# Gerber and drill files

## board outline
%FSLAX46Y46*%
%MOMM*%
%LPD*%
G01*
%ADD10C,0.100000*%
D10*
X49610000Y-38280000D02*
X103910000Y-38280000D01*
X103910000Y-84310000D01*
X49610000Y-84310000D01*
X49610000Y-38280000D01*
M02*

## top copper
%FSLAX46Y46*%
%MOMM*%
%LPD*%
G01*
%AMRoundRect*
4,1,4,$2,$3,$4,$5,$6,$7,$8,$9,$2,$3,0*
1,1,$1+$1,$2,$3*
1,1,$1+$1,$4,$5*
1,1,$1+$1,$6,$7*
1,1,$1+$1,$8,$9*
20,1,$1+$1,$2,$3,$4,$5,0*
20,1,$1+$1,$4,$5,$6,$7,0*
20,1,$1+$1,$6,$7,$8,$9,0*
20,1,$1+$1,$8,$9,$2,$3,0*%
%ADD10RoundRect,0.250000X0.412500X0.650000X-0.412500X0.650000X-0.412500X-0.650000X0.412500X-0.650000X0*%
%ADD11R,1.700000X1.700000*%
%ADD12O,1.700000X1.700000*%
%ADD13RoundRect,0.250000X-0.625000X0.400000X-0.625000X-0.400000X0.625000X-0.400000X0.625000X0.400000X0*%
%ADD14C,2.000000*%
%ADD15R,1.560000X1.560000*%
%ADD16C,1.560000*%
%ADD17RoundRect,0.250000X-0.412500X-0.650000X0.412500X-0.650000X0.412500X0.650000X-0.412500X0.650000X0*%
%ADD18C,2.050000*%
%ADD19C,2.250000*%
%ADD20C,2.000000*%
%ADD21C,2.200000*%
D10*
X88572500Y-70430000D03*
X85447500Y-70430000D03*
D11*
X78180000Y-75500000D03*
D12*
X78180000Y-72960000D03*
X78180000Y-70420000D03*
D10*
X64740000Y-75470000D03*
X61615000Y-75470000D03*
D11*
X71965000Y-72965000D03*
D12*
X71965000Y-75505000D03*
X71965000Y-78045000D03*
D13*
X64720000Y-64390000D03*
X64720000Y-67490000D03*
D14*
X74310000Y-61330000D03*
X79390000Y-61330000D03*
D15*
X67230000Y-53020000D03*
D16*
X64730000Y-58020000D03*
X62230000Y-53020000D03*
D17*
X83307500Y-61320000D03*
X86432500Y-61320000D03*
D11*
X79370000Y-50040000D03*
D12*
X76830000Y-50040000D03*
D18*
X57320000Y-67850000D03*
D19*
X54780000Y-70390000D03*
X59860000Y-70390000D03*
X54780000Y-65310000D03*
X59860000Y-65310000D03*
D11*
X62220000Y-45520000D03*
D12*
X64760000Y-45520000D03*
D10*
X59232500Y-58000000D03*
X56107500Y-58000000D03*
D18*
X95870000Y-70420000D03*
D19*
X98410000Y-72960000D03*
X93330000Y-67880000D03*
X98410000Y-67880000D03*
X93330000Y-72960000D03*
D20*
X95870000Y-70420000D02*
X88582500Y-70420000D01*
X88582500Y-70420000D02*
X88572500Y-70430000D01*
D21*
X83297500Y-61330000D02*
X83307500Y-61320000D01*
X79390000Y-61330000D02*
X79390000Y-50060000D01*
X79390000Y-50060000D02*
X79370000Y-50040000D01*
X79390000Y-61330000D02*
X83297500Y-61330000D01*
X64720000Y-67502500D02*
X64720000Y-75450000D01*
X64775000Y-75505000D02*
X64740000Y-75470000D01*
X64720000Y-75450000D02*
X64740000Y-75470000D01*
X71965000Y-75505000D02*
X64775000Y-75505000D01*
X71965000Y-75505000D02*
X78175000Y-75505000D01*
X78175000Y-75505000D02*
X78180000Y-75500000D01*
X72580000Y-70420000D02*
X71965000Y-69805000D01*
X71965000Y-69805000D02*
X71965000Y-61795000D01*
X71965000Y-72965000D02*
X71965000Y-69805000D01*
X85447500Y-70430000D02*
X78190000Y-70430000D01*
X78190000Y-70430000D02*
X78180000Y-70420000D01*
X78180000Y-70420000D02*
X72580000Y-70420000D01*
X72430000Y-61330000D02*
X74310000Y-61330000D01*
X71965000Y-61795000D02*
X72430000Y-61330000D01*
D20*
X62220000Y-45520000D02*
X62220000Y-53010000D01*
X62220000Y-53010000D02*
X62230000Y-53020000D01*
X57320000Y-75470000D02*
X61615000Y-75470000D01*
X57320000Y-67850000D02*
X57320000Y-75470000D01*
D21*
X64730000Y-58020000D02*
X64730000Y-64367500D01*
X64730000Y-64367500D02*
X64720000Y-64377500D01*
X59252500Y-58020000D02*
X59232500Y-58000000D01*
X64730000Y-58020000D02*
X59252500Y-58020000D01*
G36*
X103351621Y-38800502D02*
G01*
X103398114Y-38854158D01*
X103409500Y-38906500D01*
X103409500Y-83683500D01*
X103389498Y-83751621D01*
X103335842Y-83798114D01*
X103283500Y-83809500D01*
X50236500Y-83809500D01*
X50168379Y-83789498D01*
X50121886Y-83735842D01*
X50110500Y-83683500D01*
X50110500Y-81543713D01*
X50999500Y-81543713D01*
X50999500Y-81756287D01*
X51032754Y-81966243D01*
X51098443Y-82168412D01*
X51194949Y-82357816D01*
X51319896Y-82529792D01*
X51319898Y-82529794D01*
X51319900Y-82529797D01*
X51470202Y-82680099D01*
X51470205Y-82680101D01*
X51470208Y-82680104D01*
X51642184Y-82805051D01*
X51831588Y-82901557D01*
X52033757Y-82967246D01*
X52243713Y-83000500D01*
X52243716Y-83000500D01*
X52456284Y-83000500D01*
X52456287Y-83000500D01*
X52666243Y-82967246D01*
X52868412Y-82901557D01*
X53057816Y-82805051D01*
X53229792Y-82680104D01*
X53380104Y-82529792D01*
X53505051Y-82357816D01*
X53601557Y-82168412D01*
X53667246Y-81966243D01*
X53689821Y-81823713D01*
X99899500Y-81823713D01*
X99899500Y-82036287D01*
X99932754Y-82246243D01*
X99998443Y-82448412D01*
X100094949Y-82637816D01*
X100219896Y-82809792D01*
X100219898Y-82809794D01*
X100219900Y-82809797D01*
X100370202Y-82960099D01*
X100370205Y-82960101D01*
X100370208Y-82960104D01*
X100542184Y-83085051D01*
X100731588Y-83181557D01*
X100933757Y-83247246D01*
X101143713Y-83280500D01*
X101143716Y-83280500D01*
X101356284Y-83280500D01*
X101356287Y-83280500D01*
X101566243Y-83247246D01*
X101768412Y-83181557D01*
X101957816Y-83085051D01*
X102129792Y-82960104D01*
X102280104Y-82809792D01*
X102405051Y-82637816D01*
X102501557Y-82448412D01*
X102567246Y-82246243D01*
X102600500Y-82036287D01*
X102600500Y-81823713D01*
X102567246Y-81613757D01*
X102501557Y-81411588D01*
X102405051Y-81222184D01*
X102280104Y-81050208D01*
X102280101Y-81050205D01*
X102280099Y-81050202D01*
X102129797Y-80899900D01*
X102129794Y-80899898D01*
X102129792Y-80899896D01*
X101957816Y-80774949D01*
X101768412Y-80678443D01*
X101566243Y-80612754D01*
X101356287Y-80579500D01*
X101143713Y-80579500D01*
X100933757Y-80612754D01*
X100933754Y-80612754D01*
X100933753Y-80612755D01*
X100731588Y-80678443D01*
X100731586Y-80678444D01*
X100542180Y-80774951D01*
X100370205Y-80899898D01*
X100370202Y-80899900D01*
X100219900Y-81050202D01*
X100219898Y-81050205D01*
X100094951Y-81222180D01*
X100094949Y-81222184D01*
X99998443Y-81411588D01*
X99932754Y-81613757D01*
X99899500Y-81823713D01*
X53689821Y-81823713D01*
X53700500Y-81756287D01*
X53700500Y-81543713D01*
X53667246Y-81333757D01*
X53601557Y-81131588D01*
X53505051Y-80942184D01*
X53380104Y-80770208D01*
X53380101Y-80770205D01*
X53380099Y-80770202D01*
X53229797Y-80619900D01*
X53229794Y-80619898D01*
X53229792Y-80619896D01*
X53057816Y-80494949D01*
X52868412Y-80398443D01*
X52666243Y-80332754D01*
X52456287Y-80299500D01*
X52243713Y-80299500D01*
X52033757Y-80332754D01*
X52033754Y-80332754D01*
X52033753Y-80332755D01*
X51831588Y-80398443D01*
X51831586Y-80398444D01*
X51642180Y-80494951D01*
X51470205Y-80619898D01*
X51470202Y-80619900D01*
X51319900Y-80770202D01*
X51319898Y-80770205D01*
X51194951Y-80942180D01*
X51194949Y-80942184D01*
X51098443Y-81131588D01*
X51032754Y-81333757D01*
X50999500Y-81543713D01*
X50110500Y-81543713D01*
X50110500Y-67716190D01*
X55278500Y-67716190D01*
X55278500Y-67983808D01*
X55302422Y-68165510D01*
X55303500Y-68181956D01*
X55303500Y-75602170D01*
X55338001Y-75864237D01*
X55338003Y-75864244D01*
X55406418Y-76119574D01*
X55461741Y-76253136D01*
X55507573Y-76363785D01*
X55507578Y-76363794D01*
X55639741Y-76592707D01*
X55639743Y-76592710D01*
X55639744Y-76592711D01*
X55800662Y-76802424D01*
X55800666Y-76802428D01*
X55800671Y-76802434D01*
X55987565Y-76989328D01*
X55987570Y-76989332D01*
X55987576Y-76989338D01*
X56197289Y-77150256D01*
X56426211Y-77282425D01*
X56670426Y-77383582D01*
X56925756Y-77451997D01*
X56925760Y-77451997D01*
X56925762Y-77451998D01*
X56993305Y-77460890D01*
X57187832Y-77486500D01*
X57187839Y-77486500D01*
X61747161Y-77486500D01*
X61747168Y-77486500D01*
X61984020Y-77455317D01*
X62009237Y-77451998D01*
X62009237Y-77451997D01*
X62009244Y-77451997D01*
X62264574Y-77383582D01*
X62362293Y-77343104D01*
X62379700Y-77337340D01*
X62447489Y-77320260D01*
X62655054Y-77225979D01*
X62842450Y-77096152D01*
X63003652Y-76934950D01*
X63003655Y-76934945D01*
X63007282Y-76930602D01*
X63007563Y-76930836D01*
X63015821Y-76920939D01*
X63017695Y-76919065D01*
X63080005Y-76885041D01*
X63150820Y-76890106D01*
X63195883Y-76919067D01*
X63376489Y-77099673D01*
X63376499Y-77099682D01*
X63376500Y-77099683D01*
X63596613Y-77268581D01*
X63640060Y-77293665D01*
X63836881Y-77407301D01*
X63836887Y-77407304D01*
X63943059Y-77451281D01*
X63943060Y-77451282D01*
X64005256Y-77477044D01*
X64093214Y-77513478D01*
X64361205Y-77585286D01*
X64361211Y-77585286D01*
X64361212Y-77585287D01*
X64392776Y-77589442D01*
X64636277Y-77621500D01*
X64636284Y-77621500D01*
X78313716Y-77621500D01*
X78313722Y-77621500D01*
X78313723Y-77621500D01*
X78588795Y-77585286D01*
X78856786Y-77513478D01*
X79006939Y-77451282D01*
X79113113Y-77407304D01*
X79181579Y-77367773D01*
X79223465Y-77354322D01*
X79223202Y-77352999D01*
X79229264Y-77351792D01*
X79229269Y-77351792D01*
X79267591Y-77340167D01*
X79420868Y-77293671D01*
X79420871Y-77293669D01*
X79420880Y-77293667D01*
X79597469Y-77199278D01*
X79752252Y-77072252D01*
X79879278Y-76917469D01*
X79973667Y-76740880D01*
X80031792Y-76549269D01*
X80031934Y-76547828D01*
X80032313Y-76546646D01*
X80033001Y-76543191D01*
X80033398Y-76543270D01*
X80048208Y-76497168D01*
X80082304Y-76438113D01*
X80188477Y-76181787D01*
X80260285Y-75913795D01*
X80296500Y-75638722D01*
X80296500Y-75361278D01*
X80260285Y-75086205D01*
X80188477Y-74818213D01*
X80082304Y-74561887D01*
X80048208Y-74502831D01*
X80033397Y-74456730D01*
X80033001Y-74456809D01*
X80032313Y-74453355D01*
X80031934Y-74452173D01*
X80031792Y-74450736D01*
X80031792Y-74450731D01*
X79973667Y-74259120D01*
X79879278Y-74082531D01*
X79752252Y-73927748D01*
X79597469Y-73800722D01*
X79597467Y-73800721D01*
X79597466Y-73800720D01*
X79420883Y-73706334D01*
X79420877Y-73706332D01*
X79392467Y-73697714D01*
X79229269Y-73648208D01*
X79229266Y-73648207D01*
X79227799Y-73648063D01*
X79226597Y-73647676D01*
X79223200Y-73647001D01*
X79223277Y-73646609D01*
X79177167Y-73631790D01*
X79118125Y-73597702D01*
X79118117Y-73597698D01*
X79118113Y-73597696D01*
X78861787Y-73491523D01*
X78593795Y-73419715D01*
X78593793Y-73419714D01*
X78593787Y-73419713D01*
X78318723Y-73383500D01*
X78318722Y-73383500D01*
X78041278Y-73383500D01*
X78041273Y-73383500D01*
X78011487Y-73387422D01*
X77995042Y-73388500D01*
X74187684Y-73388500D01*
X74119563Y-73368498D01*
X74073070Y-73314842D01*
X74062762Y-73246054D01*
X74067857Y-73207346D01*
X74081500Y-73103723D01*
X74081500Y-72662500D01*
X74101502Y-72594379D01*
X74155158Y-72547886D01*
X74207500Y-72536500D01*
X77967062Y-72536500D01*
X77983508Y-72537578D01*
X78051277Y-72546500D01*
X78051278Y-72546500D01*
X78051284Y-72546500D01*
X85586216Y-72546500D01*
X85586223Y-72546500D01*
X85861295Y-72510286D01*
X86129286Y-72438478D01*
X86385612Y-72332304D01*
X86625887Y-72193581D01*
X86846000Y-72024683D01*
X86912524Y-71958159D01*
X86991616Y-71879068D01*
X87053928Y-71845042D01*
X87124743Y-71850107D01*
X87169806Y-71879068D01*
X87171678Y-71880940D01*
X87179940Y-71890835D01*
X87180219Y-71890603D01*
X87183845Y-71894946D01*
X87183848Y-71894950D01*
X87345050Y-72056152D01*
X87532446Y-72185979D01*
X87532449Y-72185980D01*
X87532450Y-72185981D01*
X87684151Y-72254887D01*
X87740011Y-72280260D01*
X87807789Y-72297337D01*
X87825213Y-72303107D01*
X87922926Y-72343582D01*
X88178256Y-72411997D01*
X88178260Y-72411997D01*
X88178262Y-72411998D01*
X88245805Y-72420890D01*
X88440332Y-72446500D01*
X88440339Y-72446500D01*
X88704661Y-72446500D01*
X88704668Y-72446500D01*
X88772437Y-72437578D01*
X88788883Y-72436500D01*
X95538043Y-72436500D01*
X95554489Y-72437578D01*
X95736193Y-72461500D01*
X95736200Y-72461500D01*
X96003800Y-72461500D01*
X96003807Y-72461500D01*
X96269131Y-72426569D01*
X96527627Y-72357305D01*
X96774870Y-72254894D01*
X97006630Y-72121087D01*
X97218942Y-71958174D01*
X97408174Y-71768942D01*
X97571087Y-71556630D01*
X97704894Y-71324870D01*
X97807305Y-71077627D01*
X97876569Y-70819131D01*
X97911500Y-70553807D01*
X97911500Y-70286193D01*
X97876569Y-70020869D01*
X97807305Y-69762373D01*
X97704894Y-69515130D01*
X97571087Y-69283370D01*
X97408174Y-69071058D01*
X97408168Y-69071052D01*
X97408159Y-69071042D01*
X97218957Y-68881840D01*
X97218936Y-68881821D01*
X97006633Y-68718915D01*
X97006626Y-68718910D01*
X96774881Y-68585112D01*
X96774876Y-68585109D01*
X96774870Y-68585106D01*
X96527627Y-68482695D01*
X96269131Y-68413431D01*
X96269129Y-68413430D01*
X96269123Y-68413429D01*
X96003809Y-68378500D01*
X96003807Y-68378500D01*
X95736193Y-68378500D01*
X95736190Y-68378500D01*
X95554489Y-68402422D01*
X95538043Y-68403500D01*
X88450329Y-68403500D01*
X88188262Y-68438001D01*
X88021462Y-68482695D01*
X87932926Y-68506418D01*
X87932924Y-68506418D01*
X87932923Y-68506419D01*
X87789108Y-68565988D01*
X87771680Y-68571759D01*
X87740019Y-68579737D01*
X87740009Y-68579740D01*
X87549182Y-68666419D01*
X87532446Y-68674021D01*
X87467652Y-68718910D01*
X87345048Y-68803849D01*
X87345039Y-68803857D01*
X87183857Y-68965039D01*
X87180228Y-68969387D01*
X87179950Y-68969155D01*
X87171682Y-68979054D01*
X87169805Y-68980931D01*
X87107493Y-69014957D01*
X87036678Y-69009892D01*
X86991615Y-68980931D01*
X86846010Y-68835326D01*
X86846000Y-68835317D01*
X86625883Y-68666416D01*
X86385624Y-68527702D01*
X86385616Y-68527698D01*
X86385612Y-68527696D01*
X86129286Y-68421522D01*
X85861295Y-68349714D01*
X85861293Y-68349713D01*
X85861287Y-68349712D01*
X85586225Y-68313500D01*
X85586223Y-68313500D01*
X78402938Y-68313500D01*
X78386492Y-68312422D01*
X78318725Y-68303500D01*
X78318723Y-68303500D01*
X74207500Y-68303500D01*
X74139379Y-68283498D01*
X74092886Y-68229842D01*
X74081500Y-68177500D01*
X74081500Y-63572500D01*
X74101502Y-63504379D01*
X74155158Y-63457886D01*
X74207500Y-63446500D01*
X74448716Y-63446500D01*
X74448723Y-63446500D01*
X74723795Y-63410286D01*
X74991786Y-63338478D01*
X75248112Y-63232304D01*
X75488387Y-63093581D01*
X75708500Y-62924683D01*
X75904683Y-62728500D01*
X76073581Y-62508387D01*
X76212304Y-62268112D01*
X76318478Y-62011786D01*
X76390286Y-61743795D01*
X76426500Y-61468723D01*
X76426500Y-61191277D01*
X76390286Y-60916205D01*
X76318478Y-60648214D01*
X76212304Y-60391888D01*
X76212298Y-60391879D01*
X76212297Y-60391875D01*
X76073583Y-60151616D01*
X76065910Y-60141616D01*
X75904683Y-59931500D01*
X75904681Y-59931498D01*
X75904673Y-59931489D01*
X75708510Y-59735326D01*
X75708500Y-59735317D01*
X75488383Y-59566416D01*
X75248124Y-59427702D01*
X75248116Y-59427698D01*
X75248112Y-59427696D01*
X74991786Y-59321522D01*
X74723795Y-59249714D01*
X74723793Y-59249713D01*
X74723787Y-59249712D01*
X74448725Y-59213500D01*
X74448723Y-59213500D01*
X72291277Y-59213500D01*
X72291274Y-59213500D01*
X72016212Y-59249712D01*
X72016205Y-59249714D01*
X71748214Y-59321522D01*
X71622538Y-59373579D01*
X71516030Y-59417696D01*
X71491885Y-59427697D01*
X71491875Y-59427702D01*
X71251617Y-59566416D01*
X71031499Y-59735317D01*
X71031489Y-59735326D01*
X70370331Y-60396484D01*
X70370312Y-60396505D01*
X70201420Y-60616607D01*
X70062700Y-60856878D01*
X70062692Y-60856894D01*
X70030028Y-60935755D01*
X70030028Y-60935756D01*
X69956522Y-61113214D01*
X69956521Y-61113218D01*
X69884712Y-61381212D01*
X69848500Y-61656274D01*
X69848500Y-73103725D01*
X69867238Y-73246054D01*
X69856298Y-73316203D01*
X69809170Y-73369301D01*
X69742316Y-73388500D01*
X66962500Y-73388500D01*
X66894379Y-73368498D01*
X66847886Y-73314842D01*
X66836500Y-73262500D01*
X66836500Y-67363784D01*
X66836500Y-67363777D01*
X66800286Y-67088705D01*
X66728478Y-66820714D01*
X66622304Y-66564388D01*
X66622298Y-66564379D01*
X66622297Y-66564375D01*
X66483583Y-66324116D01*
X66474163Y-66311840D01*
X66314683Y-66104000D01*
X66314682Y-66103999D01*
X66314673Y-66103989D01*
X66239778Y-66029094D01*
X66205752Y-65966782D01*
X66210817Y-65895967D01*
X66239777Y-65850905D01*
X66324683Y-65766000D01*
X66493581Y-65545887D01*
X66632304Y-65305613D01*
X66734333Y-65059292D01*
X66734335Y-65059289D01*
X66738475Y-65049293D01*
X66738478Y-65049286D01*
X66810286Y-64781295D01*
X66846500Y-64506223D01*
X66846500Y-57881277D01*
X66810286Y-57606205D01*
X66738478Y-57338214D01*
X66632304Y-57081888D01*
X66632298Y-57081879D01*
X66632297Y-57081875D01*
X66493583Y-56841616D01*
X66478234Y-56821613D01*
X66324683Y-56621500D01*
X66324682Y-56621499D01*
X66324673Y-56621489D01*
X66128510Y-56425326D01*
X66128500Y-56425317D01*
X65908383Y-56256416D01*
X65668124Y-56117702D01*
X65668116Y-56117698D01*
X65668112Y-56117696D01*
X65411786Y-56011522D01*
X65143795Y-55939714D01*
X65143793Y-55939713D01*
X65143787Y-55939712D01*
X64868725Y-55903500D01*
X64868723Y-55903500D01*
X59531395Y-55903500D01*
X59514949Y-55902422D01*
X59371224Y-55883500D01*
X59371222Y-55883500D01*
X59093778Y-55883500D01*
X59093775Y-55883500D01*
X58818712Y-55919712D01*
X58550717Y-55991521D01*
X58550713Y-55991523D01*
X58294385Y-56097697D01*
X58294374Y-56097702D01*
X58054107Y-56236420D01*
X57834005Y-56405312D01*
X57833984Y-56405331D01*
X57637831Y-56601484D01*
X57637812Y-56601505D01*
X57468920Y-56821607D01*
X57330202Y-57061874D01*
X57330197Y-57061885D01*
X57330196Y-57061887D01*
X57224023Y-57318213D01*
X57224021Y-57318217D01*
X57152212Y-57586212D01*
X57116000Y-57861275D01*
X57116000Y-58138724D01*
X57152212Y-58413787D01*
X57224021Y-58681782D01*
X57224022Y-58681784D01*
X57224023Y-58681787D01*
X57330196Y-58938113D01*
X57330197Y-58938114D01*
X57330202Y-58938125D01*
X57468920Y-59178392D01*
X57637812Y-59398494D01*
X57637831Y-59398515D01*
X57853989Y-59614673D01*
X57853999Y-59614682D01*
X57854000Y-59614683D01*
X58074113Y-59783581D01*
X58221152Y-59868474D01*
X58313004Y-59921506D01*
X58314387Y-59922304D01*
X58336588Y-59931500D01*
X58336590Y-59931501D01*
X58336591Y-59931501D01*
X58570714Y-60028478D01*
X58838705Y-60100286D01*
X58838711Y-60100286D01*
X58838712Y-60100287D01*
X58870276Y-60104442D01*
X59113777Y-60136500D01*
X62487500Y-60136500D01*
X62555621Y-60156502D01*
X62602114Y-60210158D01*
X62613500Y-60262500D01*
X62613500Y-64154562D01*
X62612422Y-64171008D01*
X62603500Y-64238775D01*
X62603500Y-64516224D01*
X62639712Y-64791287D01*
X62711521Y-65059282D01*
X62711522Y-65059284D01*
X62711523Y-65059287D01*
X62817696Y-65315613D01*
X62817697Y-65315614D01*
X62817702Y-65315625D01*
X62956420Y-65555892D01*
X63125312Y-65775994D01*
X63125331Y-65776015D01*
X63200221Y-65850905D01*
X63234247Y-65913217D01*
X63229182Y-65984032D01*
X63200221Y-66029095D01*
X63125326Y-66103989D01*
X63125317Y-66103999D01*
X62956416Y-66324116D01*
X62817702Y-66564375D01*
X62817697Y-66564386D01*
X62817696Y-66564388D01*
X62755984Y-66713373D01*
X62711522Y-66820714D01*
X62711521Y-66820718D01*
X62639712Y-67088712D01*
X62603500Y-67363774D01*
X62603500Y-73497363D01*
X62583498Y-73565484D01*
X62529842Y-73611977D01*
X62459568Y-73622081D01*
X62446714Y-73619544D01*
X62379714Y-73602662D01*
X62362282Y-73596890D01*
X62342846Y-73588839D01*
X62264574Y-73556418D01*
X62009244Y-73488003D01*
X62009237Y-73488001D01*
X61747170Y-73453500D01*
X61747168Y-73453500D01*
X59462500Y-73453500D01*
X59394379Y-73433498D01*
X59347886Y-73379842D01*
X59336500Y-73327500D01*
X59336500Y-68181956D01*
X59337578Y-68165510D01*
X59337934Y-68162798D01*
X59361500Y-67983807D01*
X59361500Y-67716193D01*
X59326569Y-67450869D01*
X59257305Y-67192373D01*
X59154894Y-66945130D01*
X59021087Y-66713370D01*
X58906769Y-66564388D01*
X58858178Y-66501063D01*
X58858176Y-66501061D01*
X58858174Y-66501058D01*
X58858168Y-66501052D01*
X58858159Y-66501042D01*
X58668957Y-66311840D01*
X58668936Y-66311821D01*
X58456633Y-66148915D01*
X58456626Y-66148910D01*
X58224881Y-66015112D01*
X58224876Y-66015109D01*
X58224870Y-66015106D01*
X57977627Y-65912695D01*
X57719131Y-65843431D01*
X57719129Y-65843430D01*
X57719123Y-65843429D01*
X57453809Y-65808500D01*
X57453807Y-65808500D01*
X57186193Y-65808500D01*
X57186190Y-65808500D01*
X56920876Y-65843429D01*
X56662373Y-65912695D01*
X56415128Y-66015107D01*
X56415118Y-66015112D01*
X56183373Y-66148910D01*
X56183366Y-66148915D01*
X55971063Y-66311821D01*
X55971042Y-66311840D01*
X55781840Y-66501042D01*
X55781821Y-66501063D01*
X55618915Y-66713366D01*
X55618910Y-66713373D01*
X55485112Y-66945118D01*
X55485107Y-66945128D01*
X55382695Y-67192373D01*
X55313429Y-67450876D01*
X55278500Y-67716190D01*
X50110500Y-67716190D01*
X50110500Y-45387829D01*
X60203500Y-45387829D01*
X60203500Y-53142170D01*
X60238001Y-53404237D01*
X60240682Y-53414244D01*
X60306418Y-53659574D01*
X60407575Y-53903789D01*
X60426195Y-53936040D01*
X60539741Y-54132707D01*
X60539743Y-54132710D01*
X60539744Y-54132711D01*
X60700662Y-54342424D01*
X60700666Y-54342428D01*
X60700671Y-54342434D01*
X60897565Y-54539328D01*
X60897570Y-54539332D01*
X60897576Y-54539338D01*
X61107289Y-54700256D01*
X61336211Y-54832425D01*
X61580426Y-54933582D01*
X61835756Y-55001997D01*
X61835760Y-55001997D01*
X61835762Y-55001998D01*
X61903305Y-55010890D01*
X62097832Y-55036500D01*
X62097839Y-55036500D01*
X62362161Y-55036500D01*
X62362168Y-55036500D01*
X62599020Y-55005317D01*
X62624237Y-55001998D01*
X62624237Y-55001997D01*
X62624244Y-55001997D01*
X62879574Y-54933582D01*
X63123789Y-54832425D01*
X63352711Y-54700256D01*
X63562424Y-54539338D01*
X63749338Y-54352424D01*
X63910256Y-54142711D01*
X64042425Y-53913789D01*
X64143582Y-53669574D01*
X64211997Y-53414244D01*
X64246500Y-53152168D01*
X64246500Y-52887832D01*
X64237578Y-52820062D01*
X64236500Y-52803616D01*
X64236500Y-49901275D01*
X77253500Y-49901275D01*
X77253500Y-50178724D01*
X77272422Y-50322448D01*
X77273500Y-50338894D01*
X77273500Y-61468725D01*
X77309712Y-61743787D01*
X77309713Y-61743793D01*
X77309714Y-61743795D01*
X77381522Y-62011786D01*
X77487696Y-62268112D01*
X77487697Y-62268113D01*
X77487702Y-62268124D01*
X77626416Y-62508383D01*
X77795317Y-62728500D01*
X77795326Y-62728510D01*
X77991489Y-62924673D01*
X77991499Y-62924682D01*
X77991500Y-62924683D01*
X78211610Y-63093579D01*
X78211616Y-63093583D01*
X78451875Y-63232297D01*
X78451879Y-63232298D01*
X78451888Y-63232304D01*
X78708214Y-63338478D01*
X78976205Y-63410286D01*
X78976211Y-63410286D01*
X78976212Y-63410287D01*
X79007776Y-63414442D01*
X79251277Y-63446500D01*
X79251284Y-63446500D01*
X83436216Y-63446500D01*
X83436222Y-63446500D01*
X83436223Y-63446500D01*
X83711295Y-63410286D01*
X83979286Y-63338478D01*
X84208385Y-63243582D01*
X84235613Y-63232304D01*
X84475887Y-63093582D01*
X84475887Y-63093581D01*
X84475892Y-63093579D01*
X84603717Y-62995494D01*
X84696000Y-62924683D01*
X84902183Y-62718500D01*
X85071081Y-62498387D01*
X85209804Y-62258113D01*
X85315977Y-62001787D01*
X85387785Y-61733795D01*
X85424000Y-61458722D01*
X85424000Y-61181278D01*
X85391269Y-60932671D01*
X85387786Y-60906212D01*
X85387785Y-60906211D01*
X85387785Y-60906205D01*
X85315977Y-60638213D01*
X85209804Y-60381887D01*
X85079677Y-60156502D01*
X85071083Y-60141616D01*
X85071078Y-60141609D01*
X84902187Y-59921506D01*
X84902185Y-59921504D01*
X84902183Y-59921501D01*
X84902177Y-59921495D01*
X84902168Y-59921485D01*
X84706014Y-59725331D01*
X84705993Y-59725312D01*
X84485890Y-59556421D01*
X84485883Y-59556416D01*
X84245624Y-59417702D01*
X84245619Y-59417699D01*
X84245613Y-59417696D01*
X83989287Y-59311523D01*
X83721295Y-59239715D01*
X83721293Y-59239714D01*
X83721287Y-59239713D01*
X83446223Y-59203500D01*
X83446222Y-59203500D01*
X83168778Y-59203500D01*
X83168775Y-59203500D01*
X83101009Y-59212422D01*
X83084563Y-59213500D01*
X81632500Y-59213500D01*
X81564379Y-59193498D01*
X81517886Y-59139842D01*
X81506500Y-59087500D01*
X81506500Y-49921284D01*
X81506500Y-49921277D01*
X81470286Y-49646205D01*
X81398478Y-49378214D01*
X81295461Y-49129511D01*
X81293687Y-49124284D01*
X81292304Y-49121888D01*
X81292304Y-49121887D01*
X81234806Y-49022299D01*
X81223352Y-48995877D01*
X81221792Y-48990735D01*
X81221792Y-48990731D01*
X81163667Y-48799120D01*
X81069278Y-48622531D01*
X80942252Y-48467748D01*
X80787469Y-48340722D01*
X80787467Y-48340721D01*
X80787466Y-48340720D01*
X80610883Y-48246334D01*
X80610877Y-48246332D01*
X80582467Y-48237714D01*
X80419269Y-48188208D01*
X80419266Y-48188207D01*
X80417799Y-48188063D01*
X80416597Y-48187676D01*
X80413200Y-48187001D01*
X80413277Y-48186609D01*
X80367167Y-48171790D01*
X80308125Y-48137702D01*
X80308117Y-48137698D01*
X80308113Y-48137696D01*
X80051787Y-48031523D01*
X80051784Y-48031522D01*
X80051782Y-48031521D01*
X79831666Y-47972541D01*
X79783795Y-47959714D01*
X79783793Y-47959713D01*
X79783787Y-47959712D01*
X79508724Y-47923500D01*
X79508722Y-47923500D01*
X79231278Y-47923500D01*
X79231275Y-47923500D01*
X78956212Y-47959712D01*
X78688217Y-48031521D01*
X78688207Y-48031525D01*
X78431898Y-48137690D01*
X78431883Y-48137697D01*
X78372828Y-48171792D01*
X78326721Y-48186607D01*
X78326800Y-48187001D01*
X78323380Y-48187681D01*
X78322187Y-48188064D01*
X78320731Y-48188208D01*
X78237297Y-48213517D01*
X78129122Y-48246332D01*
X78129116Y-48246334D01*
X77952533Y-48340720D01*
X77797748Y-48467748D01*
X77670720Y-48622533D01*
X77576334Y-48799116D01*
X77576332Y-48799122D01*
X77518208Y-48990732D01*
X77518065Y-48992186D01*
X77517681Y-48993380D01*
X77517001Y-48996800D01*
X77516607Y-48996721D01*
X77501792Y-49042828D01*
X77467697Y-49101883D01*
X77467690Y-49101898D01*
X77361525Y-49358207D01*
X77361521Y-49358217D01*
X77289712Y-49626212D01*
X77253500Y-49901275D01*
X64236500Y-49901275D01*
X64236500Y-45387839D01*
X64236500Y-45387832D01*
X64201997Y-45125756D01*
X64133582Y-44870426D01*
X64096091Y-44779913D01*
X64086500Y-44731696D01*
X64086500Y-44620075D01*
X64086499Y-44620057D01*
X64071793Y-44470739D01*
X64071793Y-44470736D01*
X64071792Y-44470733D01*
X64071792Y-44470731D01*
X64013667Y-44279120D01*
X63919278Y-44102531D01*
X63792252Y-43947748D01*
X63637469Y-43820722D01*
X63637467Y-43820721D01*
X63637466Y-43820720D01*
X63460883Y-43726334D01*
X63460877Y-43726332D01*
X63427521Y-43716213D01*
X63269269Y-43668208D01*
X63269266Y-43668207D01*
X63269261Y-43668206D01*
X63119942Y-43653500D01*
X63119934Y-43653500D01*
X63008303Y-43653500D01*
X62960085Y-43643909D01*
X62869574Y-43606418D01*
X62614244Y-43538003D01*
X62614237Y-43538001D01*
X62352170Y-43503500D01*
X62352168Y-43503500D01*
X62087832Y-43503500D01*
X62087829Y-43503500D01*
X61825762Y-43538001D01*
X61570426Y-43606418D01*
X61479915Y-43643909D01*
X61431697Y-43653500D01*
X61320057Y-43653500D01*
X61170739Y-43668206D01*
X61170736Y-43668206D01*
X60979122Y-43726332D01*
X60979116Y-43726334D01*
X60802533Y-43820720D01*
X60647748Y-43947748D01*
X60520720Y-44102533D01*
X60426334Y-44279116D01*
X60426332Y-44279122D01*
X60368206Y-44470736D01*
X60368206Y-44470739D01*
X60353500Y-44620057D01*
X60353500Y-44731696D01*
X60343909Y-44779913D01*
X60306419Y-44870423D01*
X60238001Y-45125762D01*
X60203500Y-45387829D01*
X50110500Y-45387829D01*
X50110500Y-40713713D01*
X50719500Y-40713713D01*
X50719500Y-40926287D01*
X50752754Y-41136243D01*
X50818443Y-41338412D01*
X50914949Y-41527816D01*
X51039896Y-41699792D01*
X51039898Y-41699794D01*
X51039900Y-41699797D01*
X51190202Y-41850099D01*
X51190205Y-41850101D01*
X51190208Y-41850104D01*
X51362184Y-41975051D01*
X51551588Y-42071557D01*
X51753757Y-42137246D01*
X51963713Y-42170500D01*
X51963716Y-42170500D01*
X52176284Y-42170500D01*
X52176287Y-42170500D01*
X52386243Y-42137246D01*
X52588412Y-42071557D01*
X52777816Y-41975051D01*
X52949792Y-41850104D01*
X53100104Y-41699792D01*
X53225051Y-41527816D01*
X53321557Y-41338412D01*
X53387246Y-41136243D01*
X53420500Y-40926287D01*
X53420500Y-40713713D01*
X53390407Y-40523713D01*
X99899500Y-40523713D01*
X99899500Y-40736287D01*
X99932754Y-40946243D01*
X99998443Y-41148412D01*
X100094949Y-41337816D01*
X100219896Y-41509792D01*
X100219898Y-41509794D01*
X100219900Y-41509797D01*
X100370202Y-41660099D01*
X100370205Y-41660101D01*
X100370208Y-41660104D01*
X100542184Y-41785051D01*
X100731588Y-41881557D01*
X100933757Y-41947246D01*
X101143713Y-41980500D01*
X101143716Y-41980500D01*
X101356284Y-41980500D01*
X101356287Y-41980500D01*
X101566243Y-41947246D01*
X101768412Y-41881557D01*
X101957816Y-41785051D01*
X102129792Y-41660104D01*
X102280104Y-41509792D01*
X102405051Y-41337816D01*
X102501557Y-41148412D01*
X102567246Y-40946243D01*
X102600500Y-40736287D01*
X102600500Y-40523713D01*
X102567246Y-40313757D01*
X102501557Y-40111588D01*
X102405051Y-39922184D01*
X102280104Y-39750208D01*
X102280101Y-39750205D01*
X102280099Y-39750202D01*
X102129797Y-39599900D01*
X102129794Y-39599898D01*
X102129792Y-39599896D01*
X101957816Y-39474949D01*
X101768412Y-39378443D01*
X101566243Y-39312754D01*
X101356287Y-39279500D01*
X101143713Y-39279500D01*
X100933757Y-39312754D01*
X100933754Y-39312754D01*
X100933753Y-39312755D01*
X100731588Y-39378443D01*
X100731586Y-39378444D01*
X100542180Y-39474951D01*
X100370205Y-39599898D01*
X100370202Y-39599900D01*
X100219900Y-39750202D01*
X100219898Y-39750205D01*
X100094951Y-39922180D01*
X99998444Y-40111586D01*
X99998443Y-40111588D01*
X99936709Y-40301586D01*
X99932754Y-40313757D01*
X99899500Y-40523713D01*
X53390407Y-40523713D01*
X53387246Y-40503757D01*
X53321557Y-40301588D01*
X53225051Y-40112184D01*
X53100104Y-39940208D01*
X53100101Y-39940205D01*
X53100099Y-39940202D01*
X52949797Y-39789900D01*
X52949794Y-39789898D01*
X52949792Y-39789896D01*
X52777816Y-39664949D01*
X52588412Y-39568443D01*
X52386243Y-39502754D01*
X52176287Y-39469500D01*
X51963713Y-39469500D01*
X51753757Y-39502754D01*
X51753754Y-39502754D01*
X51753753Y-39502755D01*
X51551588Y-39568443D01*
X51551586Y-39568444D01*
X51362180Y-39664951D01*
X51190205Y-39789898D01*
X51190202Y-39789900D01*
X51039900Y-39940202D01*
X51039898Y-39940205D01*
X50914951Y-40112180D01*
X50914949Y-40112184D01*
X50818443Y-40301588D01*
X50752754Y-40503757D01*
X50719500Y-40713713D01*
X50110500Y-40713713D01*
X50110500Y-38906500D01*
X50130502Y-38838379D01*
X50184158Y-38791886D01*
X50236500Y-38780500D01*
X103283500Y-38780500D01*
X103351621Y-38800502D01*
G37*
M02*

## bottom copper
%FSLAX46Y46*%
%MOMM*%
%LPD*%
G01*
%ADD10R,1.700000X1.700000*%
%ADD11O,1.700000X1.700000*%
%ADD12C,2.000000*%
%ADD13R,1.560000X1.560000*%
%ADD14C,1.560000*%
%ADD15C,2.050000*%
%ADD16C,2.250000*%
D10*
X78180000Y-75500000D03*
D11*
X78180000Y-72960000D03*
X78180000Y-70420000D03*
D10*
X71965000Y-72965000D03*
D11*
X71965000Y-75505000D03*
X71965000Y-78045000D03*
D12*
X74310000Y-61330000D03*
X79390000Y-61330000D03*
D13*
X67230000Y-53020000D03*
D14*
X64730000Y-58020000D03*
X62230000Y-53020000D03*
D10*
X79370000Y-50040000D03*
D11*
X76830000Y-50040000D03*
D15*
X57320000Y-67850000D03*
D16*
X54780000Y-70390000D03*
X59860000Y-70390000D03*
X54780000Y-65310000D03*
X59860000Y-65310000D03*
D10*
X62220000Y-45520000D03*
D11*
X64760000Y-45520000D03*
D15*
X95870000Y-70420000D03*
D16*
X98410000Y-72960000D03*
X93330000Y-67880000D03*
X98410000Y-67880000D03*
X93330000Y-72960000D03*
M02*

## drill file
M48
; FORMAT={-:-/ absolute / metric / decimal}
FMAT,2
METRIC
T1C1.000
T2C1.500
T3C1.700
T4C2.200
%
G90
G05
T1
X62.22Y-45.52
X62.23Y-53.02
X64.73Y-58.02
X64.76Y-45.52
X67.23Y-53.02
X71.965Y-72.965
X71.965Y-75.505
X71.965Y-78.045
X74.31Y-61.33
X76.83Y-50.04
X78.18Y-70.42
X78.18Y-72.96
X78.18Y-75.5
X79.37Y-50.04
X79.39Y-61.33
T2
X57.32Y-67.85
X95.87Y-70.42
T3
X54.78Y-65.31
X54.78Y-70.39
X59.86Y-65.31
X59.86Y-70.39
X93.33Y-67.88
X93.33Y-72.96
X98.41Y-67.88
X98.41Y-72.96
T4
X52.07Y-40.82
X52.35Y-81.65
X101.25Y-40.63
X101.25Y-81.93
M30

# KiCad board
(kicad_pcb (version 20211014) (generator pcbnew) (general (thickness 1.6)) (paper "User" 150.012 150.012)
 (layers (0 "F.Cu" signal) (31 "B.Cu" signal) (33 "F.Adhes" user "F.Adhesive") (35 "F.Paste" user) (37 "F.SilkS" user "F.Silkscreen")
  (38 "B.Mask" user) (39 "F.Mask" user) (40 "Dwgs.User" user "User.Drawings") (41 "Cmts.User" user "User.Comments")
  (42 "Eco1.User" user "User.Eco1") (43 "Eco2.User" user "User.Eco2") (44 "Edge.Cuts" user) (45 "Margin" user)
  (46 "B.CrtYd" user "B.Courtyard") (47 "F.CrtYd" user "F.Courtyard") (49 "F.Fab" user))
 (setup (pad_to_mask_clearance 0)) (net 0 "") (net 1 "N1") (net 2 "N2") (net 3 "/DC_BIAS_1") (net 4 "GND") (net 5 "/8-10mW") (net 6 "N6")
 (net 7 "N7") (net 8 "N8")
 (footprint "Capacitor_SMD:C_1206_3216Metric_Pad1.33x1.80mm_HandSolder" (layer "F.Cu") (at 87.01 70.43 180)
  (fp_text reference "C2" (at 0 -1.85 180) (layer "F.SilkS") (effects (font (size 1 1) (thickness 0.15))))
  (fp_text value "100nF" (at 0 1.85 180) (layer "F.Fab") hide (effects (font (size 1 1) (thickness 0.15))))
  (pad "1" smd roundrect (at -1.5625 0 180) (size 1.325 1.8) (layers "F.Cu" "F.Paste" "F.Mask") (roundrect_rratio 0.188679) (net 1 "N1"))
  (pad "2" smd roundrect (at 1.5625 0 180) (size 1.325 1.8) (layers "F.Cu" "F.Paste" "F.Mask") (roundrect_rratio 0.188679) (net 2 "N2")))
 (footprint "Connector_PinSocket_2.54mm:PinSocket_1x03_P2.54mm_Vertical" (layer "F.Cu") (at 78.18 75.5 180)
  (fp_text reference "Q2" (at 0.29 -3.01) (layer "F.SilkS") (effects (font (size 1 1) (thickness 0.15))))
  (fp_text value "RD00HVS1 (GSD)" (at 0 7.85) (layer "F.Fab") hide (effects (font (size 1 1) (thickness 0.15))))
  (pad "1" thru_hole rect (at 0 0 180) (size 1.7 1.7) (drill 1) (layers *.Cu *.Mask) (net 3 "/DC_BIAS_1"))
  (pad "2" thru_hole oval (at 0 2.54 180) (size 1.7 1.7) (drill 1) (layers *.Cu *.Mask) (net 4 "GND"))
  (pad "3" thru_hole oval (at 0 5.08 180) (size 1.7 1.7) (drill 1) (layers *.Cu *.Mask) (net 2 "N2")))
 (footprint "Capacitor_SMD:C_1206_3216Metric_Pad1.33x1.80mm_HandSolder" (layer "F.Cu") (at 63.1775 75.47 180)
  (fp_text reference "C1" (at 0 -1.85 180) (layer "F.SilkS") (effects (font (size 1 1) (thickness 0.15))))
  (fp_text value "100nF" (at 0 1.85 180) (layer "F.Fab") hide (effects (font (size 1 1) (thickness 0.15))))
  (pad "1" smd roundrect (at -1.5625 0 180) (size 1.325 1.8) (layers "F.Cu" "F.Paste" "F.Mask") (roundrect_rratio 0.188679)
   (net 3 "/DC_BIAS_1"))
  (pad "2" smd roundrect (at 1.5625 0 180) (size 1.325 1.8) (layers "F.Cu" "F.Paste" "F.Mask") (roundrect_rratio 0.188679) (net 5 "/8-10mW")))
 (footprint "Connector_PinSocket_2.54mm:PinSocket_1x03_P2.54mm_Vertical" (layer "F.Cu") (at 71.965 72.965)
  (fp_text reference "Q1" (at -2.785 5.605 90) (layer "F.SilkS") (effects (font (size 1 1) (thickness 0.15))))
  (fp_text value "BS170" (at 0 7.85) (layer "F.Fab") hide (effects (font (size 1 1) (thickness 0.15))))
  (pad "1" thru_hole rect locked (at 0 0) (size 1.7 1.7) (drill 1) (layers *.Cu *.Mask) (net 2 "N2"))
  (pad "2" thru_hole oval locked (at 0 2.54) (size 1.7 1.7) (drill 1) (layers *.Cu *.Mask) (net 3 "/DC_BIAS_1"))
  (pad "3" thru_hole oval locked (at 0 5.08) (size 1.7 1.7) (drill 1) (layers *.Cu *.Mask) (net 4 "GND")))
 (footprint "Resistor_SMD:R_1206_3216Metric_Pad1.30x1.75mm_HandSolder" (layer "F.Cu") (at 64.72 65.94 -90)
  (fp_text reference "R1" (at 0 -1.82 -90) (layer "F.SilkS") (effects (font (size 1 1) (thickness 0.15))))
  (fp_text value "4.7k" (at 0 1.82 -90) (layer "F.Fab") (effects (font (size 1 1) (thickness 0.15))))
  (pad "1" smd roundrect (at -1.55 0 270) (size 1.3 1.75) (layers "F.Cu" "F.Paste" "F.Mask") (roundrect_rratio 0.192308) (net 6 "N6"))
  (pad "2" smd roundrect (at 1.55 0 270) (size 1.3 1.75) (layers "F.Cu" "F.Paste" "F.Mask") (roundrect_rratio 0.192308) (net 3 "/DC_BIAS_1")))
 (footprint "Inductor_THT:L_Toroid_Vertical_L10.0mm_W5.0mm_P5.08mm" (layer "F.Cu") (at 74.31 61.33 90)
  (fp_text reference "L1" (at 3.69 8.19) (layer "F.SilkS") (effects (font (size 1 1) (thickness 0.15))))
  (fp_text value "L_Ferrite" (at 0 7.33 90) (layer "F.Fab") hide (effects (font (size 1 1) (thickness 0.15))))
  (pad "1" thru_hole circle locked (at 0 0 90) (size 2 2) (drill 1) (layers *.Cu *.Mask) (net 2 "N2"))
  (pad "2" thru_hole circle locked (at 0 5.08 90) (size 2 2) (drill 1) (layers *.Cu *.Mask) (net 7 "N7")))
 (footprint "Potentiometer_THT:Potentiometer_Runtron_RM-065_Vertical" (layer "F.Cu") (at 62.23 53.02)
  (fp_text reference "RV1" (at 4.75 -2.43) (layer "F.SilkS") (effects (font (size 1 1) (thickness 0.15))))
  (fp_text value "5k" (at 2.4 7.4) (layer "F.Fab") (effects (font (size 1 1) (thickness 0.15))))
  (pad "1" thru_hole rect (at 5 0) (size 1.56 1.56) (drill 1) (layers *.Cu *.Mask) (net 4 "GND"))
  (pad "2" thru_hole circle (at 2.5 5) (size 1.56 1.56) (drill 1) (layers *.Cu *.Mask) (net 6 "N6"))
  (pad "3" thru_hole circle (at 0 0) (size 1.56 1.56) (drill 1) (layers *.Cu *.Mask) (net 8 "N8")))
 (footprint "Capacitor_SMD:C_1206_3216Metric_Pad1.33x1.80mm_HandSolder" (layer "F.Cu") (at 84.87 61.32)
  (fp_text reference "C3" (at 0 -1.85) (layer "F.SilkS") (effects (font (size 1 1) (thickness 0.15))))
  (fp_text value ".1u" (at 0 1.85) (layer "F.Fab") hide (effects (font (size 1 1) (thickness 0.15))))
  (pad "1" smd roundrect (at -1.5625 0) (size 1.325 1.8) (layers "F.Cu" "F.Paste" "F.Mask") (roundrect_rratio 0.188679) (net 7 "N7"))
  (pad "2" smd roundrect (at 1.5625 0) (size 1.325 1.8) (layers "F.Cu" "F.Paste" "F.Mask") (roundrect_rratio 0.188679) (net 4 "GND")))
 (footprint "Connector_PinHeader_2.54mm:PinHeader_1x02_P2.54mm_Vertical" (layer "F.Cu") (at 79.37 50.04 -90)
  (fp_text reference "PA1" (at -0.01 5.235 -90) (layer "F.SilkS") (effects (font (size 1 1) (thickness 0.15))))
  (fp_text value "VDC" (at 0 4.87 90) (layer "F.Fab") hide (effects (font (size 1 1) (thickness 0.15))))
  (pad "1" thru_hole rect locked (at 0 0 270) (size 1.7 1.7) (drill 1) (layers *.Cu *.Mask) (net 7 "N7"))
  (pad "2" thru_hole oval locked (at 0 2.54 270) (size 1.7 1.7) (drill 1) (layers *.Cu *.Mask) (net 4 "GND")))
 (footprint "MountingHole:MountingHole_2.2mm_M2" (layer "F.Cu") (at 52.35 81.65)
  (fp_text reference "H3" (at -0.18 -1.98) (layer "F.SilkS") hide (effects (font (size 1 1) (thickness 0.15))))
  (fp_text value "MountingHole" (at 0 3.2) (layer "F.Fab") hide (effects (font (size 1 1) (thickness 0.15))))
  (pad "" np_thru_hole circle (at 0 0) (size 2.2 2.2) (drill 2.2) (layers *.Cu *.Mask)))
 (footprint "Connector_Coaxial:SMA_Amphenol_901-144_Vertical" (layer "F.Cu") (at 57.32 67.85)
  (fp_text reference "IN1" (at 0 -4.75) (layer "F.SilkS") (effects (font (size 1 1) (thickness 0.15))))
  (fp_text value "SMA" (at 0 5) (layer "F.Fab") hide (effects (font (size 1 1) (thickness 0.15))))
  (pad "1" thru_hole circle locked (at 0 0) (size 2.05 2.05) (drill 1.5) (layers *.Cu *.Mask) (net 5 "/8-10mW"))
  (pad "2" thru_hole circle locked (at -2.54 2.54) (size 2.25 2.25) (drill 1.7) (layers *.Cu *.Mask) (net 4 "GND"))
  (pad "2" thru_hole circle locked (at 2.54 2.54) (size 2.25 2.25) (drill 1.7) (layers *.Cu *.Mask) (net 4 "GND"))
  (pad "2" thru_hole circle locked (at -2.54 -2.54) (size 2.25 2.25) (drill 1.7) (layers *.Cu *.Mask) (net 4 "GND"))
  (pad "2" thru_hole circle locked (at 2.54 -2.54) (size 2.25 2.25) (drill 1.7) (layers *.Cu *.Mask) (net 4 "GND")))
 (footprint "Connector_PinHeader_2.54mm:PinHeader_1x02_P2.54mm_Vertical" (layer "F.Cu") (at 62.22 45.52 90)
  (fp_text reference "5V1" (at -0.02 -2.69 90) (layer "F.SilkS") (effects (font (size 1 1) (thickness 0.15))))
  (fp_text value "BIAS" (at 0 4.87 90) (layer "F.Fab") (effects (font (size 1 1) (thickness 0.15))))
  (pad "1" thru_hole rect (at 0 0 90) (size 1.7 1.7) (drill 1) (layers *.Cu *.Mask) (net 8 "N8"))
  (pad "2" thru_hole oval (at 0 2.54 90) (size 1.7 1.7) (drill 1) (layers *.Cu *.Mask) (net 4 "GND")))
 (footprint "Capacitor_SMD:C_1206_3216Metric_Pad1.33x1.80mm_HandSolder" (layer "F.Cu") (at 57.67 58 180)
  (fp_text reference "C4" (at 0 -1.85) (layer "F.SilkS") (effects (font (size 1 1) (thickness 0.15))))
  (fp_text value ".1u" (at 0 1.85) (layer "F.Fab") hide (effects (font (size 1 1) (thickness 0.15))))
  (pad "1" smd roundrect (at -1.5625 0 180) (size 1.325 1.8) (layers "F.Cu" "F.Paste" "F.Mask") (roundrect_rratio 0.188679) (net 6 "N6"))
  (pad "2" smd roundrect (at 1.5625 0 180) (size 1.325 1.8) (layers "F.Cu" "F.Paste" "F.Mask") (roundrect_rratio 0.188679) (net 4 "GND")))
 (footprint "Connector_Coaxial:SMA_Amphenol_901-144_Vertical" (layer "F.Cu") (at 95.87 70.42)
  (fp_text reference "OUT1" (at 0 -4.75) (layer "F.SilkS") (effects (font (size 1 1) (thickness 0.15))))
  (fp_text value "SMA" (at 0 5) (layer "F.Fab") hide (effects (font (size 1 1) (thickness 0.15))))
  (pad "1" thru_hole circle locked (at 0 0) (size 2.05 2.05) (drill 1.5) (layers *.Cu *.Mask) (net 1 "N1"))
  (pad "2" thru_hole circle locked (at 2.54 2.54) (size 2.25 2.25) (drill 1.7) (layers *.Cu *.Mask) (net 4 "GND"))
  (pad "2" thru_hole circle locked (at -2.54 -2.54) (size 2.25 2.25) (drill 1.7) (layers *.Cu *.Mask) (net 4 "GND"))
  (pad "2" thru_hole circle locked (at 2.54 -2.54) (size 2.25 2.25) (drill 1.7) (layers *.Cu *.Mask) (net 4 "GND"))
  (pad "2" thru_hole circle locked (at -2.54 2.54) (size 2.25 2.25) (drill 1.7) (layers *.Cu *.Mask) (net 4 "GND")))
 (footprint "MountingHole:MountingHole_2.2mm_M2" (layer "F.Cu") (at 52.07 40.82)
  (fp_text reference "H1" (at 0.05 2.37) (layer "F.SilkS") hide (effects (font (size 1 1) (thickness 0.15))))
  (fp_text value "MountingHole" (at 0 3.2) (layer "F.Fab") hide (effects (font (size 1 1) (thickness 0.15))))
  (pad "" np_thru_hole circle (at 0 0) (size 2.2 2.2) (drill 2.2) (layers *.Cu *.Mask)))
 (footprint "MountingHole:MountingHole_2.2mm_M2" (layer "F.Cu") (at 101.25 40.63)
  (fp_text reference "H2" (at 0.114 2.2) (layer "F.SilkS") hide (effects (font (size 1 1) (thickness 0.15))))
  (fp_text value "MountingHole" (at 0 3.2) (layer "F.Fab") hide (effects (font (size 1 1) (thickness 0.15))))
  (pad "" np_thru_hole circle (at 0 0) (size 2.2 2.2) (drill 2.2) (layers *.Cu *.Mask)))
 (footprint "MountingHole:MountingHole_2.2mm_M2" (layer "F.Cu") (at 101.25 81.93)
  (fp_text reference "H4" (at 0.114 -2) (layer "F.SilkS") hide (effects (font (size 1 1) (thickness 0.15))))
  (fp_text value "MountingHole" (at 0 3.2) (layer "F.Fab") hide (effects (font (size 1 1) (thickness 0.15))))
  (pad "" np_thru_hole circle (at 0 0) (size 2.2 2.2) (drill 2.2) (layers *.Cu *.Mask)))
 (gr_rect (start 49.61 38.28) (end 103.91 84.31) (layer "Edge.Cuts") (width 0.1) (fill none))
 (segment (start 95.87 70.42) (end 88.5825 70.42) (width 2) (layer "F.Cu") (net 1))
 (segment (start 88.5825 70.42) (end 88.5725 70.43) (width 2) (layer "F.Cu") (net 1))
 (segment (start 83.2975 61.33) (end 83.3075 61.32) (width 2.2) (layer "F.Cu") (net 7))
 (segment (start 79.39 61.33) (end 79.39 50.06) (width 2.2) (layer "F.Cu") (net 7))
 (segment (start 79.39 50.06) (end 79.37 50.04) (width 2.2) (layer "F.Cu") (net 7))
 (segment (start 79.39 61.33) (end 83.2975 61.33) (width 2.2) (layer "F.Cu") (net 7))
 (segment (start 64.72 67.5025) (end 64.72 75.45) (width 2.2) (layer "F.Cu") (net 3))
 (segment (start 64.775 75.505) (end 64.74 75.47) (width 2.2) (layer "F.Cu") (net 3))
 (segment (start 64.72 75.45) (end 64.74 75.47) (width 2.2) (layer "F.Cu") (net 3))
 (segment (start 71.965 75.505) (end 64.775 75.505) (width 2.2) (layer "F.Cu") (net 3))
 (segment (start 71.965 75.505) (end 78.175 75.505) (width 2.2) (layer "F.Cu") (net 3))
 (segment (start 78.175 75.505) (end 78.18 75.5) (width 2.2) (layer "F.Cu") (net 3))
 (segment (start 72.58 70.42) (end 71.965 69.805) (width 2.2) (layer "F.Cu") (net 2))
 (segment (start 71.965 69.805) (end 71.965 61.795) (width 2.2) (layer "F.Cu") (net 2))
 (segment (start 71.965 72.965) (end 71.965 69.805) (width 2.2) (layer "F.Cu") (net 2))
 (segment (start 85.4475 70.43) (end 78.19 70.43) (width 2.2) (layer "F.Cu") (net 2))
 (segment (start 78.19 70.43) (end 78.18 70.42) (width 2.2) (layer "F.Cu") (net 2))
 (segment (start 78.18 70.42) (end 72.58 70.42) (width 2.2) (layer "F.Cu") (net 2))
 (segment (start 72.43 61.33) (end 74.31 61.33) (width 2.2) (layer "F.Cu") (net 2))
 (segment (start 71.965 61.795) (end 72.43 61.33) (width 2.2) (layer "F.Cu") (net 2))
 (segment (start 62.22 45.52) (end 62.22 53.01) (width 2) (layer "F.Cu") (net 8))
 (segment (start 62.22 53.01) (end 62.23 53.02) (width 2) (layer "F.Cu") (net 8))
 (segment (start 57.32 75.47) (end 61.615 75.47) (width 2) (layer "F.Cu") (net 5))
 (segment (start 57.32 67.85) (end 57.32 75.47) (width 2) (layer "F.Cu") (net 5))
 (segment (start 64.73 58.02) (end 64.73 64.3675) (width 2.2) (layer "F.Cu") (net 6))
 (segment (start 64.73 64.3675) (end 64.72 64.3775) (width 2.2) (layer "F.Cu") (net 6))
 (segment (start 59.2525 58.02) (end 59.2325 58) (width 2.2) (layer "F.Cu") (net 6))
 (segment (start 64.73 58.02) (end 59.2525 58.02) (width 2.2) (layer "F.Cu") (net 6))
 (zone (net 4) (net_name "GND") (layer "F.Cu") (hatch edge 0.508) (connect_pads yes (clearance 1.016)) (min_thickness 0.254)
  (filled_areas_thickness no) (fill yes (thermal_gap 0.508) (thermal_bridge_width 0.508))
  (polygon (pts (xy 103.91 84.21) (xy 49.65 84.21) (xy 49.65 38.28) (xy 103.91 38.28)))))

